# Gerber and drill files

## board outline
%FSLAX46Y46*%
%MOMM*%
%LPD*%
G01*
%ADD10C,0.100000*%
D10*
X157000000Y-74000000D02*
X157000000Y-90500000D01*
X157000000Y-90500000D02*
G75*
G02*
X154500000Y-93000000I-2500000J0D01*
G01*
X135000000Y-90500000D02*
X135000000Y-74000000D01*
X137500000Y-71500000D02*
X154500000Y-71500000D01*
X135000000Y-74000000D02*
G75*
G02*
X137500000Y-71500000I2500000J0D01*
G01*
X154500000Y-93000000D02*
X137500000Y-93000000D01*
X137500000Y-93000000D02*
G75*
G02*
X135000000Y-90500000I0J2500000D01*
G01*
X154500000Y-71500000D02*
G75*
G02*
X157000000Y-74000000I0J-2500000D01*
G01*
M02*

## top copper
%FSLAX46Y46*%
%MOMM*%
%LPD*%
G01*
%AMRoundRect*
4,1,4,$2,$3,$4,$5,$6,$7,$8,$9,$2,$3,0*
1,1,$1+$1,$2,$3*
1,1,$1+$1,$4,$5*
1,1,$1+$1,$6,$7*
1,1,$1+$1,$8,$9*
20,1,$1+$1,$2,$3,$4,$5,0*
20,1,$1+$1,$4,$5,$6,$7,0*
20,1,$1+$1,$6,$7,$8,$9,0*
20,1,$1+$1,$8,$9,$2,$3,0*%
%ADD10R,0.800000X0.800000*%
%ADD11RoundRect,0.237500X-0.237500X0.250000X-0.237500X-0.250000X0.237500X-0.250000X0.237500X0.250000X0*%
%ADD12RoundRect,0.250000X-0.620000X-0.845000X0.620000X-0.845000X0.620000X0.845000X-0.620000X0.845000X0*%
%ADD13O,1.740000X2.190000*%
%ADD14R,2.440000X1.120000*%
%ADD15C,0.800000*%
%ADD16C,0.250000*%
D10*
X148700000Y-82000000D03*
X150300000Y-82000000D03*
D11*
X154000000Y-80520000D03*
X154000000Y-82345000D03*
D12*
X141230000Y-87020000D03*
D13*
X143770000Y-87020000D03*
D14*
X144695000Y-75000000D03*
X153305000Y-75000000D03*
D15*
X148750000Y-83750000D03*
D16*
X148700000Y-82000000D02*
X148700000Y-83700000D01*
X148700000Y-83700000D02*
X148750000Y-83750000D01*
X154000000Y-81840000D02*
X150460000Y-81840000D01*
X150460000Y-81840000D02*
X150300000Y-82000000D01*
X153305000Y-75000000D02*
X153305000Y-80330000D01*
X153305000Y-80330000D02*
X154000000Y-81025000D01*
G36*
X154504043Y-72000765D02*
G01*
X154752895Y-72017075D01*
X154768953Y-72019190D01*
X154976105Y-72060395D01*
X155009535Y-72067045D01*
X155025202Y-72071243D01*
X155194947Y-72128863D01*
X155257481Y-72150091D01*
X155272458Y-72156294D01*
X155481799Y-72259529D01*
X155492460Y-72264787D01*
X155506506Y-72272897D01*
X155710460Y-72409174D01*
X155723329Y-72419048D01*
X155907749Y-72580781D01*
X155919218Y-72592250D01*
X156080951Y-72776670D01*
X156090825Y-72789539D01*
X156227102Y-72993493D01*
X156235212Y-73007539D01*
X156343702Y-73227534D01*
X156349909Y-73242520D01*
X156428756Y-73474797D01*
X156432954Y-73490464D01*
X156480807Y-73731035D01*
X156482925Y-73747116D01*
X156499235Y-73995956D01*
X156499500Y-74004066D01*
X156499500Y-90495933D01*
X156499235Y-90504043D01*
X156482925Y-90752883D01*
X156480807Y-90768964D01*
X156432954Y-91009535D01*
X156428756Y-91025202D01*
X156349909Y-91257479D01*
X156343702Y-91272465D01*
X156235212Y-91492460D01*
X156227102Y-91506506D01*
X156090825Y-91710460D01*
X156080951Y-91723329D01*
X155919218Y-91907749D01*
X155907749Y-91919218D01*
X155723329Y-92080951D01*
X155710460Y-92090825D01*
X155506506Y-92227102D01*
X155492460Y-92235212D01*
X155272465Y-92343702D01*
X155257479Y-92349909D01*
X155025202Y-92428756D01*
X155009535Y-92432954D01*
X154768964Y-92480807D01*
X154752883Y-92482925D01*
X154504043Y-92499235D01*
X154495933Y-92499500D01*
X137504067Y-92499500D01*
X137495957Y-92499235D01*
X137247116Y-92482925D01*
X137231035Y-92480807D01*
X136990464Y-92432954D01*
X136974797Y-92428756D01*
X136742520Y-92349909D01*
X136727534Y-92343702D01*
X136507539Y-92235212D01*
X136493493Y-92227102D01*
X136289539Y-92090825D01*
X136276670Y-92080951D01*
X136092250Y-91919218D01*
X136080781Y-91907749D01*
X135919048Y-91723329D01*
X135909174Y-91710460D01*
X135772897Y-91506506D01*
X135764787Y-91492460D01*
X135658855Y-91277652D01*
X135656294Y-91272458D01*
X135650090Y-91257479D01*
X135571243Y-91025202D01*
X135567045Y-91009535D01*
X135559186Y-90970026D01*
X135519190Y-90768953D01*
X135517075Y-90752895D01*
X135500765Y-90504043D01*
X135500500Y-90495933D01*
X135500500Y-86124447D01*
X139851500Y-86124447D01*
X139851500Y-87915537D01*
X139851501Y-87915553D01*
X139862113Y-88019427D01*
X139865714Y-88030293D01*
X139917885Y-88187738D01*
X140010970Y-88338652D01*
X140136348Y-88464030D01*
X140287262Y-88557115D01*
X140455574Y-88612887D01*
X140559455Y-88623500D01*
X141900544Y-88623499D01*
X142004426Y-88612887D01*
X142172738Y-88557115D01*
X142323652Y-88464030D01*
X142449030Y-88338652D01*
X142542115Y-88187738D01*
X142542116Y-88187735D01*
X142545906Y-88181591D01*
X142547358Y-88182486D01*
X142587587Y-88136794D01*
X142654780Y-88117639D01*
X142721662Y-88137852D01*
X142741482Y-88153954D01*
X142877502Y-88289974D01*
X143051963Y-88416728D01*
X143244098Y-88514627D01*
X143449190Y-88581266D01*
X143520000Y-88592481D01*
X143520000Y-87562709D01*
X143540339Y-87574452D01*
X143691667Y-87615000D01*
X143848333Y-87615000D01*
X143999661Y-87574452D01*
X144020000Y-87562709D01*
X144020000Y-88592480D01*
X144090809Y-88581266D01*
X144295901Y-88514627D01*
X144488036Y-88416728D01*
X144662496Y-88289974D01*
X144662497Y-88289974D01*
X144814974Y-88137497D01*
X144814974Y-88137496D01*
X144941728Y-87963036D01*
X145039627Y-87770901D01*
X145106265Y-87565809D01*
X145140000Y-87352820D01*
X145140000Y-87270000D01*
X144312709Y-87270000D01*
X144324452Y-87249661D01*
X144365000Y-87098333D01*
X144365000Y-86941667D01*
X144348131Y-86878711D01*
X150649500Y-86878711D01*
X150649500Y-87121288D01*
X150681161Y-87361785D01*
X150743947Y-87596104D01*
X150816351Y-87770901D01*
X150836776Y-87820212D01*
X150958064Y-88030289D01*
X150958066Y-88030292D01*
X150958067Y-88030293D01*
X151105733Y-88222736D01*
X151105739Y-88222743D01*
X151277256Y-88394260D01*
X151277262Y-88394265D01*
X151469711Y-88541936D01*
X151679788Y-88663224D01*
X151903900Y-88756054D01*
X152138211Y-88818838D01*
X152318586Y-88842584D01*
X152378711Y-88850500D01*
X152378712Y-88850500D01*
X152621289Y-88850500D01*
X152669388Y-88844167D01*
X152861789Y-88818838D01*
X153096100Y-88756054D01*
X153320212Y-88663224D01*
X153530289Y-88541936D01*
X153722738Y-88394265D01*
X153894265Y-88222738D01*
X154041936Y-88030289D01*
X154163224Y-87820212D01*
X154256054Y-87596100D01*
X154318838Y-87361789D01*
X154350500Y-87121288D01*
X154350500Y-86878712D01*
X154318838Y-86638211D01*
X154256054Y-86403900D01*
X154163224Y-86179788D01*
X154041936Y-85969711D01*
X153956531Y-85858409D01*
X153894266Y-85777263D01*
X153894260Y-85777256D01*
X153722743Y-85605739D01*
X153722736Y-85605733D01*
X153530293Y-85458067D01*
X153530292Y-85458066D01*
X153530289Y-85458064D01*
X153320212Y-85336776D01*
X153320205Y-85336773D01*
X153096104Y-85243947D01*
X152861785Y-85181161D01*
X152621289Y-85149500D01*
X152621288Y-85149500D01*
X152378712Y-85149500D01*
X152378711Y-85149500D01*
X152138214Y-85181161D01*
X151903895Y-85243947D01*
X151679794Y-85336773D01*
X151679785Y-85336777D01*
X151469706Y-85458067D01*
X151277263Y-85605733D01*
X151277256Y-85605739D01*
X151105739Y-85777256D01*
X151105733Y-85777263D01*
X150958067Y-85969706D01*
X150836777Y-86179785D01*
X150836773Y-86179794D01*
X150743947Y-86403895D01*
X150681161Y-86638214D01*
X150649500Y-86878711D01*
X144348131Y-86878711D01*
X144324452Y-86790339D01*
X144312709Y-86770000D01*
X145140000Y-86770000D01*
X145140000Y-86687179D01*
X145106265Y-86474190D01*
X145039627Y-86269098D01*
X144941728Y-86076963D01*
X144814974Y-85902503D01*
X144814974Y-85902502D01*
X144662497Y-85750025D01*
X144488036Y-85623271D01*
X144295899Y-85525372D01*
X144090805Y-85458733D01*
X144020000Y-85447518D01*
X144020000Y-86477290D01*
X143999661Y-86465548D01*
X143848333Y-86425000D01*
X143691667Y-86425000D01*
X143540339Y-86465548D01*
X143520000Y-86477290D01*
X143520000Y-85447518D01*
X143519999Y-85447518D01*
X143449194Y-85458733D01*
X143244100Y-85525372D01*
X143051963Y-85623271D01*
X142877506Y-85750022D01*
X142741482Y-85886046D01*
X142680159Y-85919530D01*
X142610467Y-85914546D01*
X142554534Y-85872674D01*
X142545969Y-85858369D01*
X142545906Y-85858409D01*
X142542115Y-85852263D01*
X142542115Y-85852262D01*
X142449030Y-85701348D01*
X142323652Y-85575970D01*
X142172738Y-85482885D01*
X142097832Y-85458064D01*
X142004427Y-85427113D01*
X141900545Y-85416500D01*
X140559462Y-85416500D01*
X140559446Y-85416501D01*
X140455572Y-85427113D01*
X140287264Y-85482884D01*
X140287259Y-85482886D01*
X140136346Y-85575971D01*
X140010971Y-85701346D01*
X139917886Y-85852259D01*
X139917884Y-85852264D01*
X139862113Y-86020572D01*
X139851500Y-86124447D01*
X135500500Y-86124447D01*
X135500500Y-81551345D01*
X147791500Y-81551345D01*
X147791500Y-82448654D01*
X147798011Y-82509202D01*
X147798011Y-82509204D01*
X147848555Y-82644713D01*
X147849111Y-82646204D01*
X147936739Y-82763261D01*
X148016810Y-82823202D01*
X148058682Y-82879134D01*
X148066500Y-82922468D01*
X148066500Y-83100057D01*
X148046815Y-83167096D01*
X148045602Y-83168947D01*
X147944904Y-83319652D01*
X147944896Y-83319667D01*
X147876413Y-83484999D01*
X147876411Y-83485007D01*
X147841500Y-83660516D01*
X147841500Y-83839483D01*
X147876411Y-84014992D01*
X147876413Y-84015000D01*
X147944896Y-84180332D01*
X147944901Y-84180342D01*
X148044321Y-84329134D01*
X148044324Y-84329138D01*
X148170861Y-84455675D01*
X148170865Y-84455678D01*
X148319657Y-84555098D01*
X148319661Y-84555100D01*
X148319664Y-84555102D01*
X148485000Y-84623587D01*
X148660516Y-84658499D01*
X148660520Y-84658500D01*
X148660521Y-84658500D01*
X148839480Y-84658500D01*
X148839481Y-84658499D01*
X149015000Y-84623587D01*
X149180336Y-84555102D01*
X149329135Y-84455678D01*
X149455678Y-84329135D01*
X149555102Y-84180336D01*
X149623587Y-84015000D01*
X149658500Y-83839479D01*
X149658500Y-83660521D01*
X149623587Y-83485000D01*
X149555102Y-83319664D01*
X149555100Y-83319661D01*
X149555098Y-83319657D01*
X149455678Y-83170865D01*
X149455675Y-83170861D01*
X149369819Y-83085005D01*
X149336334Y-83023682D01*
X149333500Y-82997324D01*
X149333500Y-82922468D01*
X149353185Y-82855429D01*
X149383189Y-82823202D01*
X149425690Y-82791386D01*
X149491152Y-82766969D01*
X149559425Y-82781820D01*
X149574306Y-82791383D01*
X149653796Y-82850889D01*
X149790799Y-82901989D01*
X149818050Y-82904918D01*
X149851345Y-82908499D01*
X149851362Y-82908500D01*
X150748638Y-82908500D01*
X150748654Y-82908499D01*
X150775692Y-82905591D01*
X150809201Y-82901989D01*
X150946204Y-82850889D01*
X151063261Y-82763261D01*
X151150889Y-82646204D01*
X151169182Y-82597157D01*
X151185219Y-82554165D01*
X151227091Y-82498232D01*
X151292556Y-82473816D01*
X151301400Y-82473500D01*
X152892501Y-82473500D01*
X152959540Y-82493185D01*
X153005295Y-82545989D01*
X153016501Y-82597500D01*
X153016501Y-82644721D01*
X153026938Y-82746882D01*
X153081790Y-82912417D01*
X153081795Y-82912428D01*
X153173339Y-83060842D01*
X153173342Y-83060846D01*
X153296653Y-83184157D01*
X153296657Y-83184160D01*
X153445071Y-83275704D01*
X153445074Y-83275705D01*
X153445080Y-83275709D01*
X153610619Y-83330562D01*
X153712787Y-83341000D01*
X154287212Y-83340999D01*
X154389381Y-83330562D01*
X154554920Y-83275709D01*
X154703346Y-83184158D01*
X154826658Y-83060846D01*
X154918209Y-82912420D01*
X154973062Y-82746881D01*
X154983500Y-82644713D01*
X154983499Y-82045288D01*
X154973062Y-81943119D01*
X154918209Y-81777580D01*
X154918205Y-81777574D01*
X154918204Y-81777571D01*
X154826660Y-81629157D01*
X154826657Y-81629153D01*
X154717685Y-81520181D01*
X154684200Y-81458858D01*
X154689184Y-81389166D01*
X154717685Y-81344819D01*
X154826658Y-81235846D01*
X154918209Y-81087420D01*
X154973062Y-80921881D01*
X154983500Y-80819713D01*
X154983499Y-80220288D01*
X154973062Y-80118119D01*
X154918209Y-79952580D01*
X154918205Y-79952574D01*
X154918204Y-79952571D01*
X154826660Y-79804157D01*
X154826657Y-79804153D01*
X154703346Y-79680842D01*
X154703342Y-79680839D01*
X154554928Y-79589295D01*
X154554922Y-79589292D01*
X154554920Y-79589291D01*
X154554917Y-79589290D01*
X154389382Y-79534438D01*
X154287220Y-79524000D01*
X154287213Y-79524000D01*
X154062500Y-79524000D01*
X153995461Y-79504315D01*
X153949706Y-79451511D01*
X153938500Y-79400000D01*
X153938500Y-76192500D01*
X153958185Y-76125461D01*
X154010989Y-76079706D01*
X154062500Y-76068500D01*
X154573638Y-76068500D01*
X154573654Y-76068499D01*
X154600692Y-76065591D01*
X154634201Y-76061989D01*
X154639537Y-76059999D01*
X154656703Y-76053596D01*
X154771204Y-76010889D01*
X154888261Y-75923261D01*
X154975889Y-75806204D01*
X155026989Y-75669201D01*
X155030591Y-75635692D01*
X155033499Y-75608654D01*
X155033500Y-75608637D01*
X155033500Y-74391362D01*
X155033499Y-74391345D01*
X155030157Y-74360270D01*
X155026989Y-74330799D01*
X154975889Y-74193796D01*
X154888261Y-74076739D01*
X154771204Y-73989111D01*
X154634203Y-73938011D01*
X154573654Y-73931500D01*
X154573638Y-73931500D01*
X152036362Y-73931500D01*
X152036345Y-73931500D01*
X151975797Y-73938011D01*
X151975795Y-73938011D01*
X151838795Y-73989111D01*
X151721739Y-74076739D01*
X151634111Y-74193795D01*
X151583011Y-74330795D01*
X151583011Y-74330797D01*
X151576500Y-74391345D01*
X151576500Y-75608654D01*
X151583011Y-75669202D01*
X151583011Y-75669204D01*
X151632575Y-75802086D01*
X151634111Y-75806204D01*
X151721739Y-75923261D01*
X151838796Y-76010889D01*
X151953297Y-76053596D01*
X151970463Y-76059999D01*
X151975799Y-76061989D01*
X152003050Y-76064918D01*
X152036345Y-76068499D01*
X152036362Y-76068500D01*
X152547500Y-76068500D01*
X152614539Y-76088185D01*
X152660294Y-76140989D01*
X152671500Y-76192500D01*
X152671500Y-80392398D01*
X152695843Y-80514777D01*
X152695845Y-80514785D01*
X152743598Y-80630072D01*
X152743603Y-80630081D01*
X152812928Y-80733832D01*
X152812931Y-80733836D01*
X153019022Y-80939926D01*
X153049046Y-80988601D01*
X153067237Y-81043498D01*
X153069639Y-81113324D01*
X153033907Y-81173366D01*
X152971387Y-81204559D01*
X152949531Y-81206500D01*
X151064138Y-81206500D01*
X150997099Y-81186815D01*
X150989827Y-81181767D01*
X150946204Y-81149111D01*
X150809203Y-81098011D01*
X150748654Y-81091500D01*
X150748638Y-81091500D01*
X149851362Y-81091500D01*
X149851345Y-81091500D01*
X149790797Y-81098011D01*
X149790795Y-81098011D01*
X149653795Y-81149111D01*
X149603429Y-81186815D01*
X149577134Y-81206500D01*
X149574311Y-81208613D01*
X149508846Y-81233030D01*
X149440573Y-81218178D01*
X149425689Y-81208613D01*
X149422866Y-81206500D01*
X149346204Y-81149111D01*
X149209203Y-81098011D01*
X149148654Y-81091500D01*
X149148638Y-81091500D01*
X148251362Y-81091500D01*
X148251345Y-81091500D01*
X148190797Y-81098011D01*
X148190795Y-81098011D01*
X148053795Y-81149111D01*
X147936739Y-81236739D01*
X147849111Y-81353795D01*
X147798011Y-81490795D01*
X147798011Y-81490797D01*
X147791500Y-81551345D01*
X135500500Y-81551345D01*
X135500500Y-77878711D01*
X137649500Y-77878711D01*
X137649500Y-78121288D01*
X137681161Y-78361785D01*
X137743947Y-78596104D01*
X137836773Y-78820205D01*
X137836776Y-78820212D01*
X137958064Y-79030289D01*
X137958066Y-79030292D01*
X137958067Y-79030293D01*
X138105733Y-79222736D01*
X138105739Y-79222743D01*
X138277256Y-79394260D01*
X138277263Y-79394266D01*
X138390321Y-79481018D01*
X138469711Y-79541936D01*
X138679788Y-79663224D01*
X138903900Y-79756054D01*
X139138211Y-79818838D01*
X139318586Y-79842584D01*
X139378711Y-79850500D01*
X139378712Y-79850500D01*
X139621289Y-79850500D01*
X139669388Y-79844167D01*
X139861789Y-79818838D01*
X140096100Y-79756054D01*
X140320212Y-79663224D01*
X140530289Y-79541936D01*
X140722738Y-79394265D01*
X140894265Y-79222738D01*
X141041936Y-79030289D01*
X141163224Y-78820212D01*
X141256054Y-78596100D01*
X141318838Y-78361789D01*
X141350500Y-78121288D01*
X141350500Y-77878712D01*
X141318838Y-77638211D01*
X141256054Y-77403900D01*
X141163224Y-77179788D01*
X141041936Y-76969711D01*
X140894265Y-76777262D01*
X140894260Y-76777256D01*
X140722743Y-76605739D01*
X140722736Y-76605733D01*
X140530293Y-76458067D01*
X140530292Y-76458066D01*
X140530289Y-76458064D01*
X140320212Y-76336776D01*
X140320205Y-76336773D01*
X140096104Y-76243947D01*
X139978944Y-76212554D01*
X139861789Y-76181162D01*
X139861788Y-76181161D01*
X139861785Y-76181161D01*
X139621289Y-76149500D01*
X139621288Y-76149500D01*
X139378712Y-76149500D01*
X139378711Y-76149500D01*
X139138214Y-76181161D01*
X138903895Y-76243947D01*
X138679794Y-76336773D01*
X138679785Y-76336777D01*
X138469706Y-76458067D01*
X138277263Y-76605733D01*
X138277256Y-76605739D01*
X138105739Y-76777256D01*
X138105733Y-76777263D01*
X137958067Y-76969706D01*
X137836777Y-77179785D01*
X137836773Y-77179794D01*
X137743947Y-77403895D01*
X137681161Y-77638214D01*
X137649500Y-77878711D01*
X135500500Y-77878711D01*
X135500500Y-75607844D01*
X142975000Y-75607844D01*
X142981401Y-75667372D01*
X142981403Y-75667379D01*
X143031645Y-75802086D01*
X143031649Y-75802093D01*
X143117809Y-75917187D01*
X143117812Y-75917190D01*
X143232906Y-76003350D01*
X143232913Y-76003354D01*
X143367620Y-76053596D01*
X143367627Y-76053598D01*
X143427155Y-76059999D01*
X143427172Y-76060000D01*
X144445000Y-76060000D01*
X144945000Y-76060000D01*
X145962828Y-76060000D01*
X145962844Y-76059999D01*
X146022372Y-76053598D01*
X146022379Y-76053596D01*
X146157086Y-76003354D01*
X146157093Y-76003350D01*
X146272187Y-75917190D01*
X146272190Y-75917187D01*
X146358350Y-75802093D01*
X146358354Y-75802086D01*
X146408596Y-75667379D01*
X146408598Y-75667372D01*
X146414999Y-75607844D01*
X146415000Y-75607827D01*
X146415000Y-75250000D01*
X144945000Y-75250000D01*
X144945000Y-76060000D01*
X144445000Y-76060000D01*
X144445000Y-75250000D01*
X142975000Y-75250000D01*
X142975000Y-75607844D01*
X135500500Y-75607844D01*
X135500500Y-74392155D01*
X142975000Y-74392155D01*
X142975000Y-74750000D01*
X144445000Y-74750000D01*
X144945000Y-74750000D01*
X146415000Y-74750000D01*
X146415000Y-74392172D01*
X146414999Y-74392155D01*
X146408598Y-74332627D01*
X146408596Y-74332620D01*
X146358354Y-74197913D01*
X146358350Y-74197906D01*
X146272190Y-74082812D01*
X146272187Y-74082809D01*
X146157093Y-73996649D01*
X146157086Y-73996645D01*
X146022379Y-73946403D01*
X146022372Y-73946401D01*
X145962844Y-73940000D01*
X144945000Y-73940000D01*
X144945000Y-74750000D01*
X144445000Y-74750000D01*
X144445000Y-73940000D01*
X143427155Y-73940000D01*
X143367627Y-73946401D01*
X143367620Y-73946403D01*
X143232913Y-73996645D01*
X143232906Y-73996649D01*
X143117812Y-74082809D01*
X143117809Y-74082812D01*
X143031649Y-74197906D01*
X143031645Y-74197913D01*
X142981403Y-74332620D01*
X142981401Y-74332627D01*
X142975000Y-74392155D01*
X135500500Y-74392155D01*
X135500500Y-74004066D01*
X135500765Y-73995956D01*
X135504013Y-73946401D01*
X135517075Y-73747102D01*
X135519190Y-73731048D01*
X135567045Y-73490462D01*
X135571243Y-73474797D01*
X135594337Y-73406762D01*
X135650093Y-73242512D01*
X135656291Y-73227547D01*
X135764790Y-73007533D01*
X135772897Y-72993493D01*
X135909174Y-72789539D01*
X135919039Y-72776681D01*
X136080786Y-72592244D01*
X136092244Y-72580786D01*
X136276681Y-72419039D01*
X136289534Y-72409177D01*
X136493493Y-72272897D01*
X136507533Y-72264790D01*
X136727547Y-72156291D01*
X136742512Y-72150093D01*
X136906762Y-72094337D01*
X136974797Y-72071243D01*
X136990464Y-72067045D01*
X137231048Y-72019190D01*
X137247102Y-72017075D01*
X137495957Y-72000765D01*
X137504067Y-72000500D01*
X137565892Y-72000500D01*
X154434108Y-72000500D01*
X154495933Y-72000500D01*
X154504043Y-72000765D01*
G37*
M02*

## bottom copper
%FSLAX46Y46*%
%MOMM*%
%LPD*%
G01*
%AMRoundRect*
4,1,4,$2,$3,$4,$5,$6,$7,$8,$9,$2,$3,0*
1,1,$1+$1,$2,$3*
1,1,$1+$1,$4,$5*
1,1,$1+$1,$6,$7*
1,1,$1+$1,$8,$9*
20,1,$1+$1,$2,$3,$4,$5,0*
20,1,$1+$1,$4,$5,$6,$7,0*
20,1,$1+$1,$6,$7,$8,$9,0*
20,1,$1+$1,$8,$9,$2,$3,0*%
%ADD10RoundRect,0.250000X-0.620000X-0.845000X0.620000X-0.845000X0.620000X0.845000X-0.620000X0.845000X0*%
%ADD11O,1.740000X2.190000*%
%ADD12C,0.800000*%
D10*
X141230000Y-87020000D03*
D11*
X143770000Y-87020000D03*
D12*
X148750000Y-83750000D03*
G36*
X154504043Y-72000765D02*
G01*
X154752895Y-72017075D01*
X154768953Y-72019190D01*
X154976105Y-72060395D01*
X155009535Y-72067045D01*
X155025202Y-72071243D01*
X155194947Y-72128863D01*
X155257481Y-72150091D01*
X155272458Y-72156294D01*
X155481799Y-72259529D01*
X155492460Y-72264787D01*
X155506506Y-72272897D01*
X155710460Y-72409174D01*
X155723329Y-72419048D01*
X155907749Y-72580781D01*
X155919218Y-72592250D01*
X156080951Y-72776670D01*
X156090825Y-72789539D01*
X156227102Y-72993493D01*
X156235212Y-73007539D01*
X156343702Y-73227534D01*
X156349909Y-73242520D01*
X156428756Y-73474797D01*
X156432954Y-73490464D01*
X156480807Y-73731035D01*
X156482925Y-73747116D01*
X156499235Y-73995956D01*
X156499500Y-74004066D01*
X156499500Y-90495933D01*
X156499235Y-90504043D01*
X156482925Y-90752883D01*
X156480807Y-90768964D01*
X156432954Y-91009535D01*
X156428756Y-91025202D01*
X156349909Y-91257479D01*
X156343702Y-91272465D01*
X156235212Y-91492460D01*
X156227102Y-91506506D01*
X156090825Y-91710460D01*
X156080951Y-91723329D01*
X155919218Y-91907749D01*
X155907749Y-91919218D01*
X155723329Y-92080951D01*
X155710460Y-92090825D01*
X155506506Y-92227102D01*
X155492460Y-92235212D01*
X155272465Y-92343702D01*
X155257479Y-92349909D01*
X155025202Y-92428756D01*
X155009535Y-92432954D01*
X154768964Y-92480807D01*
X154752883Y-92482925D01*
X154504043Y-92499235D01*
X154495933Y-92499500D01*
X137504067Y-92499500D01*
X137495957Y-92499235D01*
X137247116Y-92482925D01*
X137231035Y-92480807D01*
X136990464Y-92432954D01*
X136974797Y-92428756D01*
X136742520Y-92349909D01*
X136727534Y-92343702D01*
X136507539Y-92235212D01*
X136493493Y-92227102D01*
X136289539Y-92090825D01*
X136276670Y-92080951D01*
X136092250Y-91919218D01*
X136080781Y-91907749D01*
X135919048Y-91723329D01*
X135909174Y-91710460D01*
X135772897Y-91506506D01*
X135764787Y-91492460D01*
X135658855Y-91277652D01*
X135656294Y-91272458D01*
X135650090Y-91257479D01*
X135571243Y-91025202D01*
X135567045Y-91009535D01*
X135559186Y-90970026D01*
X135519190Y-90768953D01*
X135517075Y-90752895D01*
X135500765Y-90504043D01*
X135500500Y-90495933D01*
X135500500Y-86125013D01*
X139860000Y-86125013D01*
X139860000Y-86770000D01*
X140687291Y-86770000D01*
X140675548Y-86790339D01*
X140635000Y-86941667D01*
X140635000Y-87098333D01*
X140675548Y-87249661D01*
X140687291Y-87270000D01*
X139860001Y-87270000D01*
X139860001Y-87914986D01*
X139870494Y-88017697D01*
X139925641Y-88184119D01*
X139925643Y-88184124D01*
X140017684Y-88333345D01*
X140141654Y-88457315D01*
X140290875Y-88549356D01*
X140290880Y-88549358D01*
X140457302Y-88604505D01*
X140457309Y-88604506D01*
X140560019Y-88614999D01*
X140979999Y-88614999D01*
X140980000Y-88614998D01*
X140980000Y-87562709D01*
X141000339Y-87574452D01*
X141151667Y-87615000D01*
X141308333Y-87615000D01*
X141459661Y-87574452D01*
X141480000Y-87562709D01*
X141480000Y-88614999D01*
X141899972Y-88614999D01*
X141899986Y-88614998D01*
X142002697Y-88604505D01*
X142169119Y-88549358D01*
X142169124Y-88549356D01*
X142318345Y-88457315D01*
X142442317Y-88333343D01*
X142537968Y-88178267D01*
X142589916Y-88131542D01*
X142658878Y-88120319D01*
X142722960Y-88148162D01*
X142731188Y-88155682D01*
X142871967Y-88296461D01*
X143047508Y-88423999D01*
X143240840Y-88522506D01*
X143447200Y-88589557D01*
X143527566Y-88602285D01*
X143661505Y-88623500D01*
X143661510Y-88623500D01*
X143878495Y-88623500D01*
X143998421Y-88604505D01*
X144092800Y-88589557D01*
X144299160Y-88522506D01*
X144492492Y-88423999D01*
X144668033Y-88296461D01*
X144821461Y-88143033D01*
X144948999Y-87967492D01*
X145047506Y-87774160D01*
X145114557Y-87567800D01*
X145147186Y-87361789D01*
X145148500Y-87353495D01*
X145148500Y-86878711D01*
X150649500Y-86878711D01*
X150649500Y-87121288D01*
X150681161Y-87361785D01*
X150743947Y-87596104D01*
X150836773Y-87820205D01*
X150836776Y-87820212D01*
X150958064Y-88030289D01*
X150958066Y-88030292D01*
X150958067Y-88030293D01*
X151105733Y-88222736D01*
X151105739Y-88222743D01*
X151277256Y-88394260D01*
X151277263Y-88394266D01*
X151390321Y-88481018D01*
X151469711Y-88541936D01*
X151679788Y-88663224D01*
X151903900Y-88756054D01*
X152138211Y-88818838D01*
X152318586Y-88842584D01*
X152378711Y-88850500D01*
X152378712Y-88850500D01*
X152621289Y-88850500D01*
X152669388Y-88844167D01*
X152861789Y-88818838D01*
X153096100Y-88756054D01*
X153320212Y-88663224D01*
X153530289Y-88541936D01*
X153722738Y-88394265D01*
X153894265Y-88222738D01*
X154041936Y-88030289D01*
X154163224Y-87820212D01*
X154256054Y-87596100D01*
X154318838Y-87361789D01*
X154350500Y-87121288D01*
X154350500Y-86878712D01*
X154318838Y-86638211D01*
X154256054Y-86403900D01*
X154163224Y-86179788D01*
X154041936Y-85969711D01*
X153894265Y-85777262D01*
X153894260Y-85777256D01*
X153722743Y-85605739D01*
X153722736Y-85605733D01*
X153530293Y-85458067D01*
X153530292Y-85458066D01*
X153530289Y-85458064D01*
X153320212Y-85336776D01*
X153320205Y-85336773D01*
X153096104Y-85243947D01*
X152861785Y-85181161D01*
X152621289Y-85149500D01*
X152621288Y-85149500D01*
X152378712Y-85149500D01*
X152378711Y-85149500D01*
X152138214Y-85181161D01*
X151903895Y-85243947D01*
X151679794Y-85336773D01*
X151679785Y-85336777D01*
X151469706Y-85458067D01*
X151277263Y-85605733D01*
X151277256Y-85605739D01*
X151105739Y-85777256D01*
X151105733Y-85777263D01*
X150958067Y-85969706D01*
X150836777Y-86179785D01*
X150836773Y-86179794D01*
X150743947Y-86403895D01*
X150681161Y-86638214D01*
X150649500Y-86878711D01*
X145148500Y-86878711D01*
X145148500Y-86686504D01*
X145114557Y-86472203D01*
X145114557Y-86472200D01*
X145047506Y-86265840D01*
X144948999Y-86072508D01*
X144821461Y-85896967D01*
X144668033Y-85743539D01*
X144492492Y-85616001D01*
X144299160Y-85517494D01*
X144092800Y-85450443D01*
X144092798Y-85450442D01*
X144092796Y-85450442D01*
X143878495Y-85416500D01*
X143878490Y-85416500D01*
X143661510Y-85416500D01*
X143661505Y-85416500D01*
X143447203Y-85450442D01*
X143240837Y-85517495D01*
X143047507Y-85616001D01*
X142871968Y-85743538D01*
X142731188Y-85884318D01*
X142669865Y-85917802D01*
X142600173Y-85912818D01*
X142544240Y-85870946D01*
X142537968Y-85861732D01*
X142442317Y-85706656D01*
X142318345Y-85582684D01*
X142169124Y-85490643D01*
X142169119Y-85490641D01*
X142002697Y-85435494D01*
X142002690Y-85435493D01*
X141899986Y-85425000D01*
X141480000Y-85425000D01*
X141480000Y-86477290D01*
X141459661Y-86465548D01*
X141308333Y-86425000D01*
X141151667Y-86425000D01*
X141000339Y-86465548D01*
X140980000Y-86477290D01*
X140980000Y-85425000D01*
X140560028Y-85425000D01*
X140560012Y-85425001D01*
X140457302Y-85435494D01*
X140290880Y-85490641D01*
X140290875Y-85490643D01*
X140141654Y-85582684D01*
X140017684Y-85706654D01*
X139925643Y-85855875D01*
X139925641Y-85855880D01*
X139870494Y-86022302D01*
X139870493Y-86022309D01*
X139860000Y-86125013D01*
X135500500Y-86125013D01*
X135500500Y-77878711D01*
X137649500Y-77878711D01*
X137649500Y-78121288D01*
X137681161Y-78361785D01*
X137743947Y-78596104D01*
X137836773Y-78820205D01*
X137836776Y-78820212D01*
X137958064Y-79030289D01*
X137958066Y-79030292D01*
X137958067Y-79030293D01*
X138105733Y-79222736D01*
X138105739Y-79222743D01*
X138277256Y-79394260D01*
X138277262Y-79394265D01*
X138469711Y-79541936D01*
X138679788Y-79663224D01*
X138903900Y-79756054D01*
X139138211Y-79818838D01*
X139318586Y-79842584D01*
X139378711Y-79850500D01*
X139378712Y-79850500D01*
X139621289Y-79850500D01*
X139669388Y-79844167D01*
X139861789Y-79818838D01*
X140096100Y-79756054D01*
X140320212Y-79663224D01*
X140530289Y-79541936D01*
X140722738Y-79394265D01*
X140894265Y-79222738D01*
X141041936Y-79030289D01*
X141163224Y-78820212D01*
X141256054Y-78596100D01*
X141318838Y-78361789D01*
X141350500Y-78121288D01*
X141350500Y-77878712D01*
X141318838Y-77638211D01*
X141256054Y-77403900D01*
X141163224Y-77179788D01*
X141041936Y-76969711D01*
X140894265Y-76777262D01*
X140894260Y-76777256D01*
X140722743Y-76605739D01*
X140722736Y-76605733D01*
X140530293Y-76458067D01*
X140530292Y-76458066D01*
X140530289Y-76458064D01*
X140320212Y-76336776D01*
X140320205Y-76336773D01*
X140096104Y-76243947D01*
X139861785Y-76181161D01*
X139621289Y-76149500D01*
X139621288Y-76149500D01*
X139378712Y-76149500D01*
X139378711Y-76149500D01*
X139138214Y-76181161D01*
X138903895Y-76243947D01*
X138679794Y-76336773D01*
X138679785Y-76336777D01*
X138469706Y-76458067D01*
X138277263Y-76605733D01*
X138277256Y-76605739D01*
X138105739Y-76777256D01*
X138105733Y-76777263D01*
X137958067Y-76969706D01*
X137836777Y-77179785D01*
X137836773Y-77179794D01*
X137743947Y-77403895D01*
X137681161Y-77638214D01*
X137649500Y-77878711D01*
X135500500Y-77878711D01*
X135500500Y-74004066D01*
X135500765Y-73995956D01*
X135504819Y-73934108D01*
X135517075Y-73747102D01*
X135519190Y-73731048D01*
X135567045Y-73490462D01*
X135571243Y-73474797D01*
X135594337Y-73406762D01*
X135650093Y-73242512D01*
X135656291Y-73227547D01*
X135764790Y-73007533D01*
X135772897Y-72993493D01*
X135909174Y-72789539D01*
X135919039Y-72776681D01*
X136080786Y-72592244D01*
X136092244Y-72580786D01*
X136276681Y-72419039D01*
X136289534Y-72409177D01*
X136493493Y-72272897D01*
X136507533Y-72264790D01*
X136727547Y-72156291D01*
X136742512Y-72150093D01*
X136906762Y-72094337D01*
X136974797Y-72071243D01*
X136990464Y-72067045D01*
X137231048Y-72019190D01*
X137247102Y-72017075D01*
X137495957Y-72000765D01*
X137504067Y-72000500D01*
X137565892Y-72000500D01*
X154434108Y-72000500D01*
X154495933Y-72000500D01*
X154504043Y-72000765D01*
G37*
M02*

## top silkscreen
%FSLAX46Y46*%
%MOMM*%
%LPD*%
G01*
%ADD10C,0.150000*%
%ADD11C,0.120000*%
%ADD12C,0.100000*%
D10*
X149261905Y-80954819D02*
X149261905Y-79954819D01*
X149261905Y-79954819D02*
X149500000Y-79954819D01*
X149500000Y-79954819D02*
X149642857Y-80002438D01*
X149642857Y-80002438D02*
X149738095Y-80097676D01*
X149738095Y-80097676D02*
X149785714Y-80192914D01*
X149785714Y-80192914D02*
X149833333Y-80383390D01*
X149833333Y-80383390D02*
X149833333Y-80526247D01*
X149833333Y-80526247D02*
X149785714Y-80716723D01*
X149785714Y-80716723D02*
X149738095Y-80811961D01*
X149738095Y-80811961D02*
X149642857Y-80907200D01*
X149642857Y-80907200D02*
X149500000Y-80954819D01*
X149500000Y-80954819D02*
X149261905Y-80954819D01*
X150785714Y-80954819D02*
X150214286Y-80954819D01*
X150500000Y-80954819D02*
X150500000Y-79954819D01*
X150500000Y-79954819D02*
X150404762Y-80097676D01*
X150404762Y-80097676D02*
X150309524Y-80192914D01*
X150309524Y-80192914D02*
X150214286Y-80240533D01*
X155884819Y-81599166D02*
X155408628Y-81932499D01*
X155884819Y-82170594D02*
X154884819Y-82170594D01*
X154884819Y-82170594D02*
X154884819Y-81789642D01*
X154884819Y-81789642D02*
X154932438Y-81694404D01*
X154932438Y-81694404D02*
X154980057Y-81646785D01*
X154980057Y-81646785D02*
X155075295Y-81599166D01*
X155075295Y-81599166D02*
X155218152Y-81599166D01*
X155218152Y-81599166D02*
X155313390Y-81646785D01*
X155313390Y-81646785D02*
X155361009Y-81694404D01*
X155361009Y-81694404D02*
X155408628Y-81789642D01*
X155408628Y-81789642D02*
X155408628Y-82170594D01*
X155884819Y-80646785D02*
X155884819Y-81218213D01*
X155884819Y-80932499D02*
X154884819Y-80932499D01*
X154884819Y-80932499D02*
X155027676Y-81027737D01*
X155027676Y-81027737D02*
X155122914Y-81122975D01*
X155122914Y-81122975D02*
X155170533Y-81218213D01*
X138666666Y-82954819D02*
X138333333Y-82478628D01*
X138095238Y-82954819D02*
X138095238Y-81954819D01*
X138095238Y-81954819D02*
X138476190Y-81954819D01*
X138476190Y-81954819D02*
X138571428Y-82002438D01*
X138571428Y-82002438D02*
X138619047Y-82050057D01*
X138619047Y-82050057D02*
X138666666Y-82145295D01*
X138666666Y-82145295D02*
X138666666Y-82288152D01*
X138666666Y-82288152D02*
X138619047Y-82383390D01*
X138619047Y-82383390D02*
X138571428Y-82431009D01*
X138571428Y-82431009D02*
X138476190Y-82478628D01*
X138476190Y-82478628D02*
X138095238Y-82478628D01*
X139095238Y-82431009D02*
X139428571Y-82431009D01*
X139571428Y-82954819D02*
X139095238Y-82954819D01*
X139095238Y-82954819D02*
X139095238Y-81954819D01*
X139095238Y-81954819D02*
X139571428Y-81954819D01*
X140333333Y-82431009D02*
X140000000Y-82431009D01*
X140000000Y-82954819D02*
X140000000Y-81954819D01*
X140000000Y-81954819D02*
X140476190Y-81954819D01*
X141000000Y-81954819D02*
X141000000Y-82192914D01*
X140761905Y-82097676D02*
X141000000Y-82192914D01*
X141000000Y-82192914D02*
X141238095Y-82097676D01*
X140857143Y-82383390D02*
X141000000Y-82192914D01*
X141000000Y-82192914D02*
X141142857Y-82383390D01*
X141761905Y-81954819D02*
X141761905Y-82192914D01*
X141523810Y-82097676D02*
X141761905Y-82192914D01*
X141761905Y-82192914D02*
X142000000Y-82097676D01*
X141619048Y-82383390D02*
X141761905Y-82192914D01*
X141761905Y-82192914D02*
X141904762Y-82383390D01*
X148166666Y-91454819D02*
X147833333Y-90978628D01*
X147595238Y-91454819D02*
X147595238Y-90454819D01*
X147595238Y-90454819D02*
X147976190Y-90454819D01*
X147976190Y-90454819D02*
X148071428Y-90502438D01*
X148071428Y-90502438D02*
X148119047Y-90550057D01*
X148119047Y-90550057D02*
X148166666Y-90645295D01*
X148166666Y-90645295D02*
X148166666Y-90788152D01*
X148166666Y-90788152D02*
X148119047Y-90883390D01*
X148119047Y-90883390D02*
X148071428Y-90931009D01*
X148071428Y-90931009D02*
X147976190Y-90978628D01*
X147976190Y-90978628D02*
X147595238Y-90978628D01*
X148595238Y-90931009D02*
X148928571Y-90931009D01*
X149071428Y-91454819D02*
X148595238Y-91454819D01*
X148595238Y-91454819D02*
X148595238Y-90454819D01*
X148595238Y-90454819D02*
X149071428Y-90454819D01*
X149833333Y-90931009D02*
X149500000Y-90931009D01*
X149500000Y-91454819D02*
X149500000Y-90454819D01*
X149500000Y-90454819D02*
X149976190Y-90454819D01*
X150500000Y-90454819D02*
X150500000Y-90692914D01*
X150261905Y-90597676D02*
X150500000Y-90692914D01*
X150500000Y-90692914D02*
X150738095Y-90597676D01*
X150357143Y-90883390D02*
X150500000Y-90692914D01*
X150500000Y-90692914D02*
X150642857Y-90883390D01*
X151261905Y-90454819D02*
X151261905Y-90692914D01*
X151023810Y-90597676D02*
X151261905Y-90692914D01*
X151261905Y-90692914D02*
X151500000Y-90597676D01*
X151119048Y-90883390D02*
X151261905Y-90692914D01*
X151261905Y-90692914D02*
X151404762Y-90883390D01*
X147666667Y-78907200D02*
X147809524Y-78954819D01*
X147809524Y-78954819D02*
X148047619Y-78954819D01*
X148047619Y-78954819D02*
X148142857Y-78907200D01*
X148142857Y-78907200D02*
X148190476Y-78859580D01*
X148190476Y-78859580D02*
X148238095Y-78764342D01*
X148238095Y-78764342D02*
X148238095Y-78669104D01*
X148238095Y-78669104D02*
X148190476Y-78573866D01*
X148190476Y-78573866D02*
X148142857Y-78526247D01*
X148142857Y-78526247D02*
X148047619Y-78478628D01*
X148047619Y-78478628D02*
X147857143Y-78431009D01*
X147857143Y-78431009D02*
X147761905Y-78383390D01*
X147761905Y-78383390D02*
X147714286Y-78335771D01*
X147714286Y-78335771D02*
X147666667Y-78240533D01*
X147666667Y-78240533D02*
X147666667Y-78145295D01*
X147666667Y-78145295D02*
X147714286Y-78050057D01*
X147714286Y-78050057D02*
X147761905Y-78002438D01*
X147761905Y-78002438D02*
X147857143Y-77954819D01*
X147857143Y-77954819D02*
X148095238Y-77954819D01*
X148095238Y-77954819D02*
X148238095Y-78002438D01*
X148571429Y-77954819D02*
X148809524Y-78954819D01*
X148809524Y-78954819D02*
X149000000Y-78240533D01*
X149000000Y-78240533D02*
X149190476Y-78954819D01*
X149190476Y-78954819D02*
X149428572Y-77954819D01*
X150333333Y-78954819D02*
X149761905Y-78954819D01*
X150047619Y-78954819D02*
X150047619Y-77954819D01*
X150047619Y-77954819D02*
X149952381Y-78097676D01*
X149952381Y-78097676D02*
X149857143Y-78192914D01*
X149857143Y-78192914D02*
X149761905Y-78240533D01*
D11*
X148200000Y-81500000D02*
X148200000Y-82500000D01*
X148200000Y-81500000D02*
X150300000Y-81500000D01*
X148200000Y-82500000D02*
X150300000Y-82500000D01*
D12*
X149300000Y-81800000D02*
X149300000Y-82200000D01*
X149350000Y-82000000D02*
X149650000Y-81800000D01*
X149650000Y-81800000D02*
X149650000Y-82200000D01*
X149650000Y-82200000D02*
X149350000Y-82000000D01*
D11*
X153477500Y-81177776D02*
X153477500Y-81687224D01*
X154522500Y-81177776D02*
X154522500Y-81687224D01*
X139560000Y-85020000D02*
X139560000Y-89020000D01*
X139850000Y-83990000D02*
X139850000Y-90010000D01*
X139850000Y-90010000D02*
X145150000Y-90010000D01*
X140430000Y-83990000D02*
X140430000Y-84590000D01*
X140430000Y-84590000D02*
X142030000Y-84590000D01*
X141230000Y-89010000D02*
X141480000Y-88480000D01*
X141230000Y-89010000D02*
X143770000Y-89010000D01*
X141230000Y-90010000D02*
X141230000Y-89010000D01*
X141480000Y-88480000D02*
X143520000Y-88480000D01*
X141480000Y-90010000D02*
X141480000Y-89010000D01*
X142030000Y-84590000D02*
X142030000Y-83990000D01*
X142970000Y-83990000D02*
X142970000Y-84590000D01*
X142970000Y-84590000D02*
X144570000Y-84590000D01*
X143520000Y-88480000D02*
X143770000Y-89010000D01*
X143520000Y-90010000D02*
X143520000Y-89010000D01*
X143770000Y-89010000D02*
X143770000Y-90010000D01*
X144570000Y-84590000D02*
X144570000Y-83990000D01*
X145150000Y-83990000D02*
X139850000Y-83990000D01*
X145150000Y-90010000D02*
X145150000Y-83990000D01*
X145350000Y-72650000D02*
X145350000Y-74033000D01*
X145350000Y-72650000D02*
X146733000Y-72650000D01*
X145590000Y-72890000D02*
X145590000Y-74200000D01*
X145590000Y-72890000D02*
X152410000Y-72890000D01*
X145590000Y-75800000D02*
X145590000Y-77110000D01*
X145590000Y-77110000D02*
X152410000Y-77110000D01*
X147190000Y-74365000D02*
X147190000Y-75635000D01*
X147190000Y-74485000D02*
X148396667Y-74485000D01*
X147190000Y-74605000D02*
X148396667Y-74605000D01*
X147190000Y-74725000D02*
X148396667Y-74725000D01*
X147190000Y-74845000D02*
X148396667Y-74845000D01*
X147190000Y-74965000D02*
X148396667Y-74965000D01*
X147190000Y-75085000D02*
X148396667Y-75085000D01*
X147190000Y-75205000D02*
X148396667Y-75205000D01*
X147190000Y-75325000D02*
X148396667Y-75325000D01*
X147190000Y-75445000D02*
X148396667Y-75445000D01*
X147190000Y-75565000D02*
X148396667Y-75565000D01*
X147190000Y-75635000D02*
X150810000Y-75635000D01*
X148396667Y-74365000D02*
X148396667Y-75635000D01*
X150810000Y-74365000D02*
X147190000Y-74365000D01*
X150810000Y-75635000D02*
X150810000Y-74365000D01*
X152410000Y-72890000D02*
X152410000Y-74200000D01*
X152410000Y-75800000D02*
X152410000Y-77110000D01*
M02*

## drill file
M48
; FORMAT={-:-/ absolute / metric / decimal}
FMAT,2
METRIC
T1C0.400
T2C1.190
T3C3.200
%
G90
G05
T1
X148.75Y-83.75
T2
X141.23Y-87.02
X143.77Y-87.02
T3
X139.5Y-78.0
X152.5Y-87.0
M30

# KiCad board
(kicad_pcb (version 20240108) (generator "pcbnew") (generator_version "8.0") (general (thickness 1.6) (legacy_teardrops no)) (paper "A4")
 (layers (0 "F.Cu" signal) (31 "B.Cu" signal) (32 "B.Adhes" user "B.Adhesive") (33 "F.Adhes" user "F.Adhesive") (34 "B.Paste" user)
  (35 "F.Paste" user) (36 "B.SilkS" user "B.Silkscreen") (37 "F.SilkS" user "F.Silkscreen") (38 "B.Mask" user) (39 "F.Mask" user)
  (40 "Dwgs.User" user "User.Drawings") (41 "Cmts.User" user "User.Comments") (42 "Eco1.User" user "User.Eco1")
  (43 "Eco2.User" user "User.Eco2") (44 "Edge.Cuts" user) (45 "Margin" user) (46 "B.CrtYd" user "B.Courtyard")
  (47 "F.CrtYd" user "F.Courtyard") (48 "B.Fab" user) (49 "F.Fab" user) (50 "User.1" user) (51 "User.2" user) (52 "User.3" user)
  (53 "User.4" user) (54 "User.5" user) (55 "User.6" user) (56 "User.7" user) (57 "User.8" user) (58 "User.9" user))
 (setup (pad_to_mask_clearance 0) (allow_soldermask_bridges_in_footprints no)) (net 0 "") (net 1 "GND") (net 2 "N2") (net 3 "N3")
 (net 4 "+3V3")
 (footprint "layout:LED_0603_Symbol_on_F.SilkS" (layer "F.Cu") (at 149.5 82)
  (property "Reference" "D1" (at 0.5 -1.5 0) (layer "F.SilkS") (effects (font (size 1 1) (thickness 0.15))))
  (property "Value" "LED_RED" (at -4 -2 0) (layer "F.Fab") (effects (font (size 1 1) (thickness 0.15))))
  (fp_line (start -1.3 -0.5) (end -1.3 0.5) (stroke (width 0.12) (type solid)) (layer "F.SilkS"))
  (fp_line (start -1.3 -0.5) (end 0.8 -0.5) (stroke (width 0.12) (type solid)) (layer "F.SilkS"))
  (fp_line (start -1.3 0.5) (end 0.8 0.5) (stroke (width 0.12) (type solid)) (layer "F.SilkS"))
  (fp_line (start -0.2 -0.2) (end -0.2 0.2) (stroke (width 0.1) (type solid)) (layer "F.SilkS"))
  (fp_line (start -0.15 0) (end 0.15 -0.2) (stroke (width 0.1) (type solid)) (layer "F.SilkS"))
  (fp_line (start 0.15 -0.2) (end 0.15 0.2) (stroke (width 0.1) (type solid)) (layer "F.SilkS"))
  (fp_line (start 0.15 0.2) (end -0.15 0) (stroke (width 0.1) (type solid)) (layer "F.SilkS"))
  (pad "1" smd rect (at -0.8 0 180) (size 0.8 0.8) (layers "F.Cu" "F.Paste" "F.Mask") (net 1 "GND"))
  (pad "2" smd rect (at 0.8 0 180) (size 0.8 0.8) (layers "F.Cu" "F.Paste" "F.Mask") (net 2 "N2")))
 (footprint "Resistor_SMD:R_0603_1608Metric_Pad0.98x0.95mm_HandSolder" (layer "F.Cu") (at 154 81.4325 -90)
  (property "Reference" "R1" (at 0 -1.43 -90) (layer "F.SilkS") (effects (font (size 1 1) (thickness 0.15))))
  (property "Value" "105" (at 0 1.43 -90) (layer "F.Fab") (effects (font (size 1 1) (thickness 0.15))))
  (fp_line (start -0.254724 0.5225) (end 0.254724 0.5225) (stroke (width 0.12) (type solid)) (layer "F.SilkS"))
  (fp_line (start -0.254724 -0.5225) (end 0.254724 -0.5225) (stroke (width 0.12) (type solid)) (layer "F.SilkS"))
  (pad "1" smd roundrect (at -0.9125 0 270) (size 0.975 0.95) (layers "F.Cu" "F.Paste" "F.Mask") (roundrect_rratio 0.25) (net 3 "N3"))
  (pad "2" smd roundrect (at 0.9125 0 270) (size 0.975 0.95) (layers "F.Cu" "F.Paste" "F.Mask") (roundrect_rratio 0.25) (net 2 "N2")))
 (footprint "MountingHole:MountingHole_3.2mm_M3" (layer "F.Cu") (at 139.5 78)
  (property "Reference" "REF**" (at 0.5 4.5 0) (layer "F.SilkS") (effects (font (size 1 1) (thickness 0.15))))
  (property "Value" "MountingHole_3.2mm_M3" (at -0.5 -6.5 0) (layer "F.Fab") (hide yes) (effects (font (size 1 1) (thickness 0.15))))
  (pad "" np_thru_hole circle (at 0 0) (size 3.2 3.2) (drill 3.2) (layers "*.Cu" "*.Mask")))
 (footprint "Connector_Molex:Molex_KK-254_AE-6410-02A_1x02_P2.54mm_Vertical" (layer "F.Cu") (at 141.23 87.02)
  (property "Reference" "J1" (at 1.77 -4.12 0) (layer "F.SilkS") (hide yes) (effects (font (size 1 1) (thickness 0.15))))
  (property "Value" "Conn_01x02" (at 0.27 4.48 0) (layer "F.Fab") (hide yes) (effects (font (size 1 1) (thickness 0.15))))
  (fp_line (start -1.67 -2) (end -1.67 2) (stroke (width 0.12) (type solid)) (layer "F.SilkS"))
  (fp_line (start -1.38 -3.03) (end -1.38 2.99) (stroke (width 0.12) (type solid)) (layer "F.SilkS"))
  (fp_line (start -1.38 2.99) (end 3.92 2.99) (stroke (width 0.12) (type solid)) (layer "F.SilkS"))
  (fp_line (start -0.8 -3.03) (end -0.8 -2.43) (stroke (width 0.12) (type solid)) (layer "F.SilkS"))
  (fp_line (start -0.8 -2.43) (end 0.8 -2.43) (stroke (width 0.12) (type solid)) (layer "F.SilkS"))
  (fp_line (start 0 1.99) (end 0.25 1.46) (stroke (width 0.12) (type solid)) (layer "F.SilkS"))
  (fp_line (start 0 1.99) (end 2.54 1.99) (stroke (width 0.12) (type solid)) (layer "F.SilkS"))
  (fp_line (start 0 2.99) (end 0 1.99) (stroke (width 0.12) (type solid)) (layer "F.SilkS"))
  (fp_line (start 0.25 1.46) (end 2.29 1.46) (stroke (width 0.12) (type solid)) (layer "F.SilkS"))
  (fp_line (start 0.25 2.99) (end 0.25 1.99) (stroke (width 0.12) (type solid)) (layer "F.SilkS"))
  (fp_line (start 0.8 -2.43) (end 0.8 -3.03) (stroke (width 0.12) (type solid)) (layer "F.SilkS"))
  (fp_line (start 1.74 -3.03) (end 1.74 -2.43) (stroke (width 0.12) (type solid)) (layer "F.SilkS"))
  (fp_line (start 1.74 -2.43) (end 3.34 -2.43) (stroke (width 0.12) (type solid)) (layer "F.SilkS"))
  (fp_line (start 2.29 1.46) (end 2.54 1.99) (stroke (width 0.12) (type solid)) (layer "F.SilkS"))
  (fp_line (start 2.29 2.99) (end 2.29 1.99) (stroke (width 0.12) (type solid)) (layer "F.SilkS"))
  (fp_line (start 2.54 1.99) (end 2.54 2.99) (stroke (width 0.12) (type solid)) (layer "F.SilkS"))
  (fp_line (start 3.34 -2.43) (end 3.34 -3.03) (stroke (width 0.12) (type solid)) (layer "F.SilkS"))
  (fp_line (start 3.92 -3.03) (end -1.38 -3.03) (stroke (width 0.12) (type solid)) (layer "F.SilkS"))
  (fp_line (start 3.92 2.99) (end 3.92 -3.03) (stroke (width 0.12) (type solid)) (layer "F.SilkS"))
  (pad "1" thru_hole roundrect (at 0 0) (size 1.74 2.19) (drill 1.19) (layers "*.Cu" "*.Mask") (remove_unused_layers no)
   (roundrect_rratio 0.143678) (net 1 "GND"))
  (pad "2" thru_hole oval (at 2.54 0) (size 1.74 2.19) (drill 1.19) (layers "*.Cu" "*.Mask") (remove_unused_layers no) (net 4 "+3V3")))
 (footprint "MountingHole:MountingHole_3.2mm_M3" (layer "F.Cu") (at 152.5 87)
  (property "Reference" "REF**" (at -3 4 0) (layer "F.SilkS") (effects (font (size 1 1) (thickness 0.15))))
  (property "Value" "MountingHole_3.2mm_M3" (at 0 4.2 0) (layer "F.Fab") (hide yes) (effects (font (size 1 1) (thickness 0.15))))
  (pad "" np_thru_hole circle (at 0 0) (size 3.2 3.2) (drill 3.2) (layers "*.Cu" "*.Mask")))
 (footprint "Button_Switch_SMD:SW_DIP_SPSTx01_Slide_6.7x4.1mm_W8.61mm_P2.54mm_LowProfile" (layer "F.Cu") (at 149 75)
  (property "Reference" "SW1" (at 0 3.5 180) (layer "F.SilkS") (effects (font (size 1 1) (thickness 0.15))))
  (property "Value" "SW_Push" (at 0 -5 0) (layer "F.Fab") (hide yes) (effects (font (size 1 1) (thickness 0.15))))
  (fp_line (start -3.65 -2.35) (end -3.65 -0.967) (stroke (width 0.12) (type solid)) (layer "F.SilkS"))
  (fp_line (start -3.65 -2.35) (end -2.267 -2.35) (stroke (width 0.12) (type solid)) (layer "F.SilkS"))
  (fp_line (start -3.41 -2.11) (end -3.41 -0.8) (stroke (width 0.12) (type solid)) (layer "F.SilkS"))
  (fp_line (start -3.41 -2.11) (end 3.41 -2.11) (stroke (width 0.12) (type solid)) (layer "F.SilkS"))
  (fp_line (start -3.41 0.8) (end -3.41 2.11) (stroke (width 0.12) (type solid)) (layer "F.SilkS"))
  (fp_line (start -3.41 2.11) (end 3.41 2.11) (stroke (width 0.12) (type solid)) (layer "F.SilkS"))
  (fp_line (start -1.81 -0.635) (end -1.81 0.635) (stroke (width 0.12) (type solid)) (layer "F.SilkS"))
  (fp_line (start -1.81 -0.515) (end -0.603333 -0.515) (stroke (width 0.12) (type solid)) (layer "F.SilkS"))
  (fp_line (start -1.81 -0.395) (end -0.603333 -0.395) (stroke (width 0.12) (type solid)) (layer "F.SilkS"))
  (fp_line (start -1.81 -0.275) (end -0.603333 -0.275) (stroke (width 0.12) (type solid)) (layer "F.SilkS"))
  (fp_line (start -1.81 -0.155) (end -0.603333 -0.155) (stroke (width 0.12) (type solid)) (layer "F.SilkS"))
  (fp_line (start -1.81 -0.035) (end -0.603333 -0.035) (stroke (width 0.12) (type solid)) (layer "F.SilkS"))
  (fp_line (start -1.81 0.085) (end -0.603333 0.085) (stroke (width 0.12) (type solid)) (layer "F.SilkS"))
  (fp_line (start -1.81 0.205) (end -0.603333 0.205) (stroke (width 0.12) (type solid)) (layer "F.SilkS"))
  (fp_line (start -1.81 0.325) (end -0.603333 0.325) (stroke (width 0.12) (type solid)) (layer "F.SilkS"))
  (fp_line (start -1.81 0.445) (end -0.603333 0.445) (stroke (width 0.12) (type solid)) (layer "F.SilkS"))
  (fp_line (start -1.81 0.565) (end -0.603333 0.565) (stroke (width 0.12) (type solid)) (layer "F.SilkS"))
  (fp_line (start -1.81 0.635) (end 1.81 0.635) (stroke (width 0.12) (type solid)) (layer "F.SilkS"))
  (fp_line (start -0.603333 -0.635) (end -0.603333 0.635) (stroke (width 0.12) (type solid)) (layer "F.SilkS"))
  (fp_line (start 1.81 -0.635) (end -1.81 -0.635) (stroke (width 0.12) (type solid)) (layer "F.SilkS"))
  (fp_line (start 1.81 0.635) (end 1.81 -0.635) (stroke (width 0.12) (type solid)) (layer "F.SilkS"))
  (fp_line (start 3.41 -2.11) (end 3.41 -0.8) (stroke (width 0.12) (type solid)) (layer "F.SilkS"))
  (fp_line (start 3.41 0.8) (end 3.41 2.11) (stroke (width 0.12) (type solid)) (layer "F.SilkS"))
  (pad "1" smd rect (at -4.305 0) (size 2.44 1.12) (layers "F.Cu" "F.Paste" "F.Mask") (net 4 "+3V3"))
  (pad "2" smd rect (at 4.305 0) (size 2.44 1.12) (layers "F.Cu" "F.Paste" "F.Mask") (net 3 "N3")))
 (gr_line (start 157 74) (end 157 90.5) (stroke (width 0.1) (type default)) (layer "Edge.Cuts"))
 (gr_arc (start 157 90.5) (mid 156.267767 92.267767) (end 154.5 93) (stroke (width 0.1) (type default)) (layer "Edge.Cuts"))
 (gr_line (start 135 90.5) (end 135 74) (stroke (width 0.1) (type default)) (layer "Edge.Cuts"))
 (gr_line (start 137.5 71.5) (end 154.5 71.5) (stroke (width 0.1) (type default)) (layer "Edge.Cuts"))
 (gr_arc (start 135 74) (mid 135.732233 72.232233) (end 137.5 71.5) (stroke (width 0.1) (type default)) (layer "Edge.Cuts"))
 (gr_line (start 154.5 93) (end 137.5 93) (stroke (width 0.1) (type default)) (layer "Edge.Cuts"))
 (gr_arc (start 137.5 93) (mid 135.732233 92.267767) (end 135 90.5) (stroke (width 0.1) (type default)) (layer "Edge.Cuts"))
 (gr_arc (start 154.5 71.5) (mid 156.267767 72.232233) (end 157 74) (stroke (width 0.1) (type default)) (layer "Edge.Cuts"))
 (segment (start 148.7 82) (end 148.7 83.7) (width 0.25) (layer "F.Cu") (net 1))
 (segment (start 148.7 83.7) (end 148.75 83.75) (width 0.25) (layer "F.Cu") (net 1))
 (via (at 148.75 83.75) (size 0.8) (drill 0.4) (layers "F.Cu" "B.Cu") (free yes) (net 1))
 (segment (start 154 81.84) (end 150.46 81.84) (width 0.25) (layer "F.Cu") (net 2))
 (segment (start 150.46 81.84) (end 150.3 82) (width 0.25) (layer "F.Cu") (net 2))
 (segment (start 153.305 75) (end 153.305 80.33) (width 0.25) (layer "F.Cu") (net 3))
 (segment (start 153.305 80.33) (end 154 81.025) (width 0.25) (layer "F.Cu") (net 3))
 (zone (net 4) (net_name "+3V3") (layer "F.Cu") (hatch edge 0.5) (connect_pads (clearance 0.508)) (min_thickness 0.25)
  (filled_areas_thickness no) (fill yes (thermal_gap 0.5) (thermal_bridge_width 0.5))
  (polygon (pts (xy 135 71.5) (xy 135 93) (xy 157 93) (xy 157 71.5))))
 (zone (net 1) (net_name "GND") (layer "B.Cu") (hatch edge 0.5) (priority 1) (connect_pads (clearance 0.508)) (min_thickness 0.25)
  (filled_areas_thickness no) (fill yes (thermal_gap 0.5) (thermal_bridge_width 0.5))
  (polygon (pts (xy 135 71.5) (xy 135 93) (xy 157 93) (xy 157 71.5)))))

